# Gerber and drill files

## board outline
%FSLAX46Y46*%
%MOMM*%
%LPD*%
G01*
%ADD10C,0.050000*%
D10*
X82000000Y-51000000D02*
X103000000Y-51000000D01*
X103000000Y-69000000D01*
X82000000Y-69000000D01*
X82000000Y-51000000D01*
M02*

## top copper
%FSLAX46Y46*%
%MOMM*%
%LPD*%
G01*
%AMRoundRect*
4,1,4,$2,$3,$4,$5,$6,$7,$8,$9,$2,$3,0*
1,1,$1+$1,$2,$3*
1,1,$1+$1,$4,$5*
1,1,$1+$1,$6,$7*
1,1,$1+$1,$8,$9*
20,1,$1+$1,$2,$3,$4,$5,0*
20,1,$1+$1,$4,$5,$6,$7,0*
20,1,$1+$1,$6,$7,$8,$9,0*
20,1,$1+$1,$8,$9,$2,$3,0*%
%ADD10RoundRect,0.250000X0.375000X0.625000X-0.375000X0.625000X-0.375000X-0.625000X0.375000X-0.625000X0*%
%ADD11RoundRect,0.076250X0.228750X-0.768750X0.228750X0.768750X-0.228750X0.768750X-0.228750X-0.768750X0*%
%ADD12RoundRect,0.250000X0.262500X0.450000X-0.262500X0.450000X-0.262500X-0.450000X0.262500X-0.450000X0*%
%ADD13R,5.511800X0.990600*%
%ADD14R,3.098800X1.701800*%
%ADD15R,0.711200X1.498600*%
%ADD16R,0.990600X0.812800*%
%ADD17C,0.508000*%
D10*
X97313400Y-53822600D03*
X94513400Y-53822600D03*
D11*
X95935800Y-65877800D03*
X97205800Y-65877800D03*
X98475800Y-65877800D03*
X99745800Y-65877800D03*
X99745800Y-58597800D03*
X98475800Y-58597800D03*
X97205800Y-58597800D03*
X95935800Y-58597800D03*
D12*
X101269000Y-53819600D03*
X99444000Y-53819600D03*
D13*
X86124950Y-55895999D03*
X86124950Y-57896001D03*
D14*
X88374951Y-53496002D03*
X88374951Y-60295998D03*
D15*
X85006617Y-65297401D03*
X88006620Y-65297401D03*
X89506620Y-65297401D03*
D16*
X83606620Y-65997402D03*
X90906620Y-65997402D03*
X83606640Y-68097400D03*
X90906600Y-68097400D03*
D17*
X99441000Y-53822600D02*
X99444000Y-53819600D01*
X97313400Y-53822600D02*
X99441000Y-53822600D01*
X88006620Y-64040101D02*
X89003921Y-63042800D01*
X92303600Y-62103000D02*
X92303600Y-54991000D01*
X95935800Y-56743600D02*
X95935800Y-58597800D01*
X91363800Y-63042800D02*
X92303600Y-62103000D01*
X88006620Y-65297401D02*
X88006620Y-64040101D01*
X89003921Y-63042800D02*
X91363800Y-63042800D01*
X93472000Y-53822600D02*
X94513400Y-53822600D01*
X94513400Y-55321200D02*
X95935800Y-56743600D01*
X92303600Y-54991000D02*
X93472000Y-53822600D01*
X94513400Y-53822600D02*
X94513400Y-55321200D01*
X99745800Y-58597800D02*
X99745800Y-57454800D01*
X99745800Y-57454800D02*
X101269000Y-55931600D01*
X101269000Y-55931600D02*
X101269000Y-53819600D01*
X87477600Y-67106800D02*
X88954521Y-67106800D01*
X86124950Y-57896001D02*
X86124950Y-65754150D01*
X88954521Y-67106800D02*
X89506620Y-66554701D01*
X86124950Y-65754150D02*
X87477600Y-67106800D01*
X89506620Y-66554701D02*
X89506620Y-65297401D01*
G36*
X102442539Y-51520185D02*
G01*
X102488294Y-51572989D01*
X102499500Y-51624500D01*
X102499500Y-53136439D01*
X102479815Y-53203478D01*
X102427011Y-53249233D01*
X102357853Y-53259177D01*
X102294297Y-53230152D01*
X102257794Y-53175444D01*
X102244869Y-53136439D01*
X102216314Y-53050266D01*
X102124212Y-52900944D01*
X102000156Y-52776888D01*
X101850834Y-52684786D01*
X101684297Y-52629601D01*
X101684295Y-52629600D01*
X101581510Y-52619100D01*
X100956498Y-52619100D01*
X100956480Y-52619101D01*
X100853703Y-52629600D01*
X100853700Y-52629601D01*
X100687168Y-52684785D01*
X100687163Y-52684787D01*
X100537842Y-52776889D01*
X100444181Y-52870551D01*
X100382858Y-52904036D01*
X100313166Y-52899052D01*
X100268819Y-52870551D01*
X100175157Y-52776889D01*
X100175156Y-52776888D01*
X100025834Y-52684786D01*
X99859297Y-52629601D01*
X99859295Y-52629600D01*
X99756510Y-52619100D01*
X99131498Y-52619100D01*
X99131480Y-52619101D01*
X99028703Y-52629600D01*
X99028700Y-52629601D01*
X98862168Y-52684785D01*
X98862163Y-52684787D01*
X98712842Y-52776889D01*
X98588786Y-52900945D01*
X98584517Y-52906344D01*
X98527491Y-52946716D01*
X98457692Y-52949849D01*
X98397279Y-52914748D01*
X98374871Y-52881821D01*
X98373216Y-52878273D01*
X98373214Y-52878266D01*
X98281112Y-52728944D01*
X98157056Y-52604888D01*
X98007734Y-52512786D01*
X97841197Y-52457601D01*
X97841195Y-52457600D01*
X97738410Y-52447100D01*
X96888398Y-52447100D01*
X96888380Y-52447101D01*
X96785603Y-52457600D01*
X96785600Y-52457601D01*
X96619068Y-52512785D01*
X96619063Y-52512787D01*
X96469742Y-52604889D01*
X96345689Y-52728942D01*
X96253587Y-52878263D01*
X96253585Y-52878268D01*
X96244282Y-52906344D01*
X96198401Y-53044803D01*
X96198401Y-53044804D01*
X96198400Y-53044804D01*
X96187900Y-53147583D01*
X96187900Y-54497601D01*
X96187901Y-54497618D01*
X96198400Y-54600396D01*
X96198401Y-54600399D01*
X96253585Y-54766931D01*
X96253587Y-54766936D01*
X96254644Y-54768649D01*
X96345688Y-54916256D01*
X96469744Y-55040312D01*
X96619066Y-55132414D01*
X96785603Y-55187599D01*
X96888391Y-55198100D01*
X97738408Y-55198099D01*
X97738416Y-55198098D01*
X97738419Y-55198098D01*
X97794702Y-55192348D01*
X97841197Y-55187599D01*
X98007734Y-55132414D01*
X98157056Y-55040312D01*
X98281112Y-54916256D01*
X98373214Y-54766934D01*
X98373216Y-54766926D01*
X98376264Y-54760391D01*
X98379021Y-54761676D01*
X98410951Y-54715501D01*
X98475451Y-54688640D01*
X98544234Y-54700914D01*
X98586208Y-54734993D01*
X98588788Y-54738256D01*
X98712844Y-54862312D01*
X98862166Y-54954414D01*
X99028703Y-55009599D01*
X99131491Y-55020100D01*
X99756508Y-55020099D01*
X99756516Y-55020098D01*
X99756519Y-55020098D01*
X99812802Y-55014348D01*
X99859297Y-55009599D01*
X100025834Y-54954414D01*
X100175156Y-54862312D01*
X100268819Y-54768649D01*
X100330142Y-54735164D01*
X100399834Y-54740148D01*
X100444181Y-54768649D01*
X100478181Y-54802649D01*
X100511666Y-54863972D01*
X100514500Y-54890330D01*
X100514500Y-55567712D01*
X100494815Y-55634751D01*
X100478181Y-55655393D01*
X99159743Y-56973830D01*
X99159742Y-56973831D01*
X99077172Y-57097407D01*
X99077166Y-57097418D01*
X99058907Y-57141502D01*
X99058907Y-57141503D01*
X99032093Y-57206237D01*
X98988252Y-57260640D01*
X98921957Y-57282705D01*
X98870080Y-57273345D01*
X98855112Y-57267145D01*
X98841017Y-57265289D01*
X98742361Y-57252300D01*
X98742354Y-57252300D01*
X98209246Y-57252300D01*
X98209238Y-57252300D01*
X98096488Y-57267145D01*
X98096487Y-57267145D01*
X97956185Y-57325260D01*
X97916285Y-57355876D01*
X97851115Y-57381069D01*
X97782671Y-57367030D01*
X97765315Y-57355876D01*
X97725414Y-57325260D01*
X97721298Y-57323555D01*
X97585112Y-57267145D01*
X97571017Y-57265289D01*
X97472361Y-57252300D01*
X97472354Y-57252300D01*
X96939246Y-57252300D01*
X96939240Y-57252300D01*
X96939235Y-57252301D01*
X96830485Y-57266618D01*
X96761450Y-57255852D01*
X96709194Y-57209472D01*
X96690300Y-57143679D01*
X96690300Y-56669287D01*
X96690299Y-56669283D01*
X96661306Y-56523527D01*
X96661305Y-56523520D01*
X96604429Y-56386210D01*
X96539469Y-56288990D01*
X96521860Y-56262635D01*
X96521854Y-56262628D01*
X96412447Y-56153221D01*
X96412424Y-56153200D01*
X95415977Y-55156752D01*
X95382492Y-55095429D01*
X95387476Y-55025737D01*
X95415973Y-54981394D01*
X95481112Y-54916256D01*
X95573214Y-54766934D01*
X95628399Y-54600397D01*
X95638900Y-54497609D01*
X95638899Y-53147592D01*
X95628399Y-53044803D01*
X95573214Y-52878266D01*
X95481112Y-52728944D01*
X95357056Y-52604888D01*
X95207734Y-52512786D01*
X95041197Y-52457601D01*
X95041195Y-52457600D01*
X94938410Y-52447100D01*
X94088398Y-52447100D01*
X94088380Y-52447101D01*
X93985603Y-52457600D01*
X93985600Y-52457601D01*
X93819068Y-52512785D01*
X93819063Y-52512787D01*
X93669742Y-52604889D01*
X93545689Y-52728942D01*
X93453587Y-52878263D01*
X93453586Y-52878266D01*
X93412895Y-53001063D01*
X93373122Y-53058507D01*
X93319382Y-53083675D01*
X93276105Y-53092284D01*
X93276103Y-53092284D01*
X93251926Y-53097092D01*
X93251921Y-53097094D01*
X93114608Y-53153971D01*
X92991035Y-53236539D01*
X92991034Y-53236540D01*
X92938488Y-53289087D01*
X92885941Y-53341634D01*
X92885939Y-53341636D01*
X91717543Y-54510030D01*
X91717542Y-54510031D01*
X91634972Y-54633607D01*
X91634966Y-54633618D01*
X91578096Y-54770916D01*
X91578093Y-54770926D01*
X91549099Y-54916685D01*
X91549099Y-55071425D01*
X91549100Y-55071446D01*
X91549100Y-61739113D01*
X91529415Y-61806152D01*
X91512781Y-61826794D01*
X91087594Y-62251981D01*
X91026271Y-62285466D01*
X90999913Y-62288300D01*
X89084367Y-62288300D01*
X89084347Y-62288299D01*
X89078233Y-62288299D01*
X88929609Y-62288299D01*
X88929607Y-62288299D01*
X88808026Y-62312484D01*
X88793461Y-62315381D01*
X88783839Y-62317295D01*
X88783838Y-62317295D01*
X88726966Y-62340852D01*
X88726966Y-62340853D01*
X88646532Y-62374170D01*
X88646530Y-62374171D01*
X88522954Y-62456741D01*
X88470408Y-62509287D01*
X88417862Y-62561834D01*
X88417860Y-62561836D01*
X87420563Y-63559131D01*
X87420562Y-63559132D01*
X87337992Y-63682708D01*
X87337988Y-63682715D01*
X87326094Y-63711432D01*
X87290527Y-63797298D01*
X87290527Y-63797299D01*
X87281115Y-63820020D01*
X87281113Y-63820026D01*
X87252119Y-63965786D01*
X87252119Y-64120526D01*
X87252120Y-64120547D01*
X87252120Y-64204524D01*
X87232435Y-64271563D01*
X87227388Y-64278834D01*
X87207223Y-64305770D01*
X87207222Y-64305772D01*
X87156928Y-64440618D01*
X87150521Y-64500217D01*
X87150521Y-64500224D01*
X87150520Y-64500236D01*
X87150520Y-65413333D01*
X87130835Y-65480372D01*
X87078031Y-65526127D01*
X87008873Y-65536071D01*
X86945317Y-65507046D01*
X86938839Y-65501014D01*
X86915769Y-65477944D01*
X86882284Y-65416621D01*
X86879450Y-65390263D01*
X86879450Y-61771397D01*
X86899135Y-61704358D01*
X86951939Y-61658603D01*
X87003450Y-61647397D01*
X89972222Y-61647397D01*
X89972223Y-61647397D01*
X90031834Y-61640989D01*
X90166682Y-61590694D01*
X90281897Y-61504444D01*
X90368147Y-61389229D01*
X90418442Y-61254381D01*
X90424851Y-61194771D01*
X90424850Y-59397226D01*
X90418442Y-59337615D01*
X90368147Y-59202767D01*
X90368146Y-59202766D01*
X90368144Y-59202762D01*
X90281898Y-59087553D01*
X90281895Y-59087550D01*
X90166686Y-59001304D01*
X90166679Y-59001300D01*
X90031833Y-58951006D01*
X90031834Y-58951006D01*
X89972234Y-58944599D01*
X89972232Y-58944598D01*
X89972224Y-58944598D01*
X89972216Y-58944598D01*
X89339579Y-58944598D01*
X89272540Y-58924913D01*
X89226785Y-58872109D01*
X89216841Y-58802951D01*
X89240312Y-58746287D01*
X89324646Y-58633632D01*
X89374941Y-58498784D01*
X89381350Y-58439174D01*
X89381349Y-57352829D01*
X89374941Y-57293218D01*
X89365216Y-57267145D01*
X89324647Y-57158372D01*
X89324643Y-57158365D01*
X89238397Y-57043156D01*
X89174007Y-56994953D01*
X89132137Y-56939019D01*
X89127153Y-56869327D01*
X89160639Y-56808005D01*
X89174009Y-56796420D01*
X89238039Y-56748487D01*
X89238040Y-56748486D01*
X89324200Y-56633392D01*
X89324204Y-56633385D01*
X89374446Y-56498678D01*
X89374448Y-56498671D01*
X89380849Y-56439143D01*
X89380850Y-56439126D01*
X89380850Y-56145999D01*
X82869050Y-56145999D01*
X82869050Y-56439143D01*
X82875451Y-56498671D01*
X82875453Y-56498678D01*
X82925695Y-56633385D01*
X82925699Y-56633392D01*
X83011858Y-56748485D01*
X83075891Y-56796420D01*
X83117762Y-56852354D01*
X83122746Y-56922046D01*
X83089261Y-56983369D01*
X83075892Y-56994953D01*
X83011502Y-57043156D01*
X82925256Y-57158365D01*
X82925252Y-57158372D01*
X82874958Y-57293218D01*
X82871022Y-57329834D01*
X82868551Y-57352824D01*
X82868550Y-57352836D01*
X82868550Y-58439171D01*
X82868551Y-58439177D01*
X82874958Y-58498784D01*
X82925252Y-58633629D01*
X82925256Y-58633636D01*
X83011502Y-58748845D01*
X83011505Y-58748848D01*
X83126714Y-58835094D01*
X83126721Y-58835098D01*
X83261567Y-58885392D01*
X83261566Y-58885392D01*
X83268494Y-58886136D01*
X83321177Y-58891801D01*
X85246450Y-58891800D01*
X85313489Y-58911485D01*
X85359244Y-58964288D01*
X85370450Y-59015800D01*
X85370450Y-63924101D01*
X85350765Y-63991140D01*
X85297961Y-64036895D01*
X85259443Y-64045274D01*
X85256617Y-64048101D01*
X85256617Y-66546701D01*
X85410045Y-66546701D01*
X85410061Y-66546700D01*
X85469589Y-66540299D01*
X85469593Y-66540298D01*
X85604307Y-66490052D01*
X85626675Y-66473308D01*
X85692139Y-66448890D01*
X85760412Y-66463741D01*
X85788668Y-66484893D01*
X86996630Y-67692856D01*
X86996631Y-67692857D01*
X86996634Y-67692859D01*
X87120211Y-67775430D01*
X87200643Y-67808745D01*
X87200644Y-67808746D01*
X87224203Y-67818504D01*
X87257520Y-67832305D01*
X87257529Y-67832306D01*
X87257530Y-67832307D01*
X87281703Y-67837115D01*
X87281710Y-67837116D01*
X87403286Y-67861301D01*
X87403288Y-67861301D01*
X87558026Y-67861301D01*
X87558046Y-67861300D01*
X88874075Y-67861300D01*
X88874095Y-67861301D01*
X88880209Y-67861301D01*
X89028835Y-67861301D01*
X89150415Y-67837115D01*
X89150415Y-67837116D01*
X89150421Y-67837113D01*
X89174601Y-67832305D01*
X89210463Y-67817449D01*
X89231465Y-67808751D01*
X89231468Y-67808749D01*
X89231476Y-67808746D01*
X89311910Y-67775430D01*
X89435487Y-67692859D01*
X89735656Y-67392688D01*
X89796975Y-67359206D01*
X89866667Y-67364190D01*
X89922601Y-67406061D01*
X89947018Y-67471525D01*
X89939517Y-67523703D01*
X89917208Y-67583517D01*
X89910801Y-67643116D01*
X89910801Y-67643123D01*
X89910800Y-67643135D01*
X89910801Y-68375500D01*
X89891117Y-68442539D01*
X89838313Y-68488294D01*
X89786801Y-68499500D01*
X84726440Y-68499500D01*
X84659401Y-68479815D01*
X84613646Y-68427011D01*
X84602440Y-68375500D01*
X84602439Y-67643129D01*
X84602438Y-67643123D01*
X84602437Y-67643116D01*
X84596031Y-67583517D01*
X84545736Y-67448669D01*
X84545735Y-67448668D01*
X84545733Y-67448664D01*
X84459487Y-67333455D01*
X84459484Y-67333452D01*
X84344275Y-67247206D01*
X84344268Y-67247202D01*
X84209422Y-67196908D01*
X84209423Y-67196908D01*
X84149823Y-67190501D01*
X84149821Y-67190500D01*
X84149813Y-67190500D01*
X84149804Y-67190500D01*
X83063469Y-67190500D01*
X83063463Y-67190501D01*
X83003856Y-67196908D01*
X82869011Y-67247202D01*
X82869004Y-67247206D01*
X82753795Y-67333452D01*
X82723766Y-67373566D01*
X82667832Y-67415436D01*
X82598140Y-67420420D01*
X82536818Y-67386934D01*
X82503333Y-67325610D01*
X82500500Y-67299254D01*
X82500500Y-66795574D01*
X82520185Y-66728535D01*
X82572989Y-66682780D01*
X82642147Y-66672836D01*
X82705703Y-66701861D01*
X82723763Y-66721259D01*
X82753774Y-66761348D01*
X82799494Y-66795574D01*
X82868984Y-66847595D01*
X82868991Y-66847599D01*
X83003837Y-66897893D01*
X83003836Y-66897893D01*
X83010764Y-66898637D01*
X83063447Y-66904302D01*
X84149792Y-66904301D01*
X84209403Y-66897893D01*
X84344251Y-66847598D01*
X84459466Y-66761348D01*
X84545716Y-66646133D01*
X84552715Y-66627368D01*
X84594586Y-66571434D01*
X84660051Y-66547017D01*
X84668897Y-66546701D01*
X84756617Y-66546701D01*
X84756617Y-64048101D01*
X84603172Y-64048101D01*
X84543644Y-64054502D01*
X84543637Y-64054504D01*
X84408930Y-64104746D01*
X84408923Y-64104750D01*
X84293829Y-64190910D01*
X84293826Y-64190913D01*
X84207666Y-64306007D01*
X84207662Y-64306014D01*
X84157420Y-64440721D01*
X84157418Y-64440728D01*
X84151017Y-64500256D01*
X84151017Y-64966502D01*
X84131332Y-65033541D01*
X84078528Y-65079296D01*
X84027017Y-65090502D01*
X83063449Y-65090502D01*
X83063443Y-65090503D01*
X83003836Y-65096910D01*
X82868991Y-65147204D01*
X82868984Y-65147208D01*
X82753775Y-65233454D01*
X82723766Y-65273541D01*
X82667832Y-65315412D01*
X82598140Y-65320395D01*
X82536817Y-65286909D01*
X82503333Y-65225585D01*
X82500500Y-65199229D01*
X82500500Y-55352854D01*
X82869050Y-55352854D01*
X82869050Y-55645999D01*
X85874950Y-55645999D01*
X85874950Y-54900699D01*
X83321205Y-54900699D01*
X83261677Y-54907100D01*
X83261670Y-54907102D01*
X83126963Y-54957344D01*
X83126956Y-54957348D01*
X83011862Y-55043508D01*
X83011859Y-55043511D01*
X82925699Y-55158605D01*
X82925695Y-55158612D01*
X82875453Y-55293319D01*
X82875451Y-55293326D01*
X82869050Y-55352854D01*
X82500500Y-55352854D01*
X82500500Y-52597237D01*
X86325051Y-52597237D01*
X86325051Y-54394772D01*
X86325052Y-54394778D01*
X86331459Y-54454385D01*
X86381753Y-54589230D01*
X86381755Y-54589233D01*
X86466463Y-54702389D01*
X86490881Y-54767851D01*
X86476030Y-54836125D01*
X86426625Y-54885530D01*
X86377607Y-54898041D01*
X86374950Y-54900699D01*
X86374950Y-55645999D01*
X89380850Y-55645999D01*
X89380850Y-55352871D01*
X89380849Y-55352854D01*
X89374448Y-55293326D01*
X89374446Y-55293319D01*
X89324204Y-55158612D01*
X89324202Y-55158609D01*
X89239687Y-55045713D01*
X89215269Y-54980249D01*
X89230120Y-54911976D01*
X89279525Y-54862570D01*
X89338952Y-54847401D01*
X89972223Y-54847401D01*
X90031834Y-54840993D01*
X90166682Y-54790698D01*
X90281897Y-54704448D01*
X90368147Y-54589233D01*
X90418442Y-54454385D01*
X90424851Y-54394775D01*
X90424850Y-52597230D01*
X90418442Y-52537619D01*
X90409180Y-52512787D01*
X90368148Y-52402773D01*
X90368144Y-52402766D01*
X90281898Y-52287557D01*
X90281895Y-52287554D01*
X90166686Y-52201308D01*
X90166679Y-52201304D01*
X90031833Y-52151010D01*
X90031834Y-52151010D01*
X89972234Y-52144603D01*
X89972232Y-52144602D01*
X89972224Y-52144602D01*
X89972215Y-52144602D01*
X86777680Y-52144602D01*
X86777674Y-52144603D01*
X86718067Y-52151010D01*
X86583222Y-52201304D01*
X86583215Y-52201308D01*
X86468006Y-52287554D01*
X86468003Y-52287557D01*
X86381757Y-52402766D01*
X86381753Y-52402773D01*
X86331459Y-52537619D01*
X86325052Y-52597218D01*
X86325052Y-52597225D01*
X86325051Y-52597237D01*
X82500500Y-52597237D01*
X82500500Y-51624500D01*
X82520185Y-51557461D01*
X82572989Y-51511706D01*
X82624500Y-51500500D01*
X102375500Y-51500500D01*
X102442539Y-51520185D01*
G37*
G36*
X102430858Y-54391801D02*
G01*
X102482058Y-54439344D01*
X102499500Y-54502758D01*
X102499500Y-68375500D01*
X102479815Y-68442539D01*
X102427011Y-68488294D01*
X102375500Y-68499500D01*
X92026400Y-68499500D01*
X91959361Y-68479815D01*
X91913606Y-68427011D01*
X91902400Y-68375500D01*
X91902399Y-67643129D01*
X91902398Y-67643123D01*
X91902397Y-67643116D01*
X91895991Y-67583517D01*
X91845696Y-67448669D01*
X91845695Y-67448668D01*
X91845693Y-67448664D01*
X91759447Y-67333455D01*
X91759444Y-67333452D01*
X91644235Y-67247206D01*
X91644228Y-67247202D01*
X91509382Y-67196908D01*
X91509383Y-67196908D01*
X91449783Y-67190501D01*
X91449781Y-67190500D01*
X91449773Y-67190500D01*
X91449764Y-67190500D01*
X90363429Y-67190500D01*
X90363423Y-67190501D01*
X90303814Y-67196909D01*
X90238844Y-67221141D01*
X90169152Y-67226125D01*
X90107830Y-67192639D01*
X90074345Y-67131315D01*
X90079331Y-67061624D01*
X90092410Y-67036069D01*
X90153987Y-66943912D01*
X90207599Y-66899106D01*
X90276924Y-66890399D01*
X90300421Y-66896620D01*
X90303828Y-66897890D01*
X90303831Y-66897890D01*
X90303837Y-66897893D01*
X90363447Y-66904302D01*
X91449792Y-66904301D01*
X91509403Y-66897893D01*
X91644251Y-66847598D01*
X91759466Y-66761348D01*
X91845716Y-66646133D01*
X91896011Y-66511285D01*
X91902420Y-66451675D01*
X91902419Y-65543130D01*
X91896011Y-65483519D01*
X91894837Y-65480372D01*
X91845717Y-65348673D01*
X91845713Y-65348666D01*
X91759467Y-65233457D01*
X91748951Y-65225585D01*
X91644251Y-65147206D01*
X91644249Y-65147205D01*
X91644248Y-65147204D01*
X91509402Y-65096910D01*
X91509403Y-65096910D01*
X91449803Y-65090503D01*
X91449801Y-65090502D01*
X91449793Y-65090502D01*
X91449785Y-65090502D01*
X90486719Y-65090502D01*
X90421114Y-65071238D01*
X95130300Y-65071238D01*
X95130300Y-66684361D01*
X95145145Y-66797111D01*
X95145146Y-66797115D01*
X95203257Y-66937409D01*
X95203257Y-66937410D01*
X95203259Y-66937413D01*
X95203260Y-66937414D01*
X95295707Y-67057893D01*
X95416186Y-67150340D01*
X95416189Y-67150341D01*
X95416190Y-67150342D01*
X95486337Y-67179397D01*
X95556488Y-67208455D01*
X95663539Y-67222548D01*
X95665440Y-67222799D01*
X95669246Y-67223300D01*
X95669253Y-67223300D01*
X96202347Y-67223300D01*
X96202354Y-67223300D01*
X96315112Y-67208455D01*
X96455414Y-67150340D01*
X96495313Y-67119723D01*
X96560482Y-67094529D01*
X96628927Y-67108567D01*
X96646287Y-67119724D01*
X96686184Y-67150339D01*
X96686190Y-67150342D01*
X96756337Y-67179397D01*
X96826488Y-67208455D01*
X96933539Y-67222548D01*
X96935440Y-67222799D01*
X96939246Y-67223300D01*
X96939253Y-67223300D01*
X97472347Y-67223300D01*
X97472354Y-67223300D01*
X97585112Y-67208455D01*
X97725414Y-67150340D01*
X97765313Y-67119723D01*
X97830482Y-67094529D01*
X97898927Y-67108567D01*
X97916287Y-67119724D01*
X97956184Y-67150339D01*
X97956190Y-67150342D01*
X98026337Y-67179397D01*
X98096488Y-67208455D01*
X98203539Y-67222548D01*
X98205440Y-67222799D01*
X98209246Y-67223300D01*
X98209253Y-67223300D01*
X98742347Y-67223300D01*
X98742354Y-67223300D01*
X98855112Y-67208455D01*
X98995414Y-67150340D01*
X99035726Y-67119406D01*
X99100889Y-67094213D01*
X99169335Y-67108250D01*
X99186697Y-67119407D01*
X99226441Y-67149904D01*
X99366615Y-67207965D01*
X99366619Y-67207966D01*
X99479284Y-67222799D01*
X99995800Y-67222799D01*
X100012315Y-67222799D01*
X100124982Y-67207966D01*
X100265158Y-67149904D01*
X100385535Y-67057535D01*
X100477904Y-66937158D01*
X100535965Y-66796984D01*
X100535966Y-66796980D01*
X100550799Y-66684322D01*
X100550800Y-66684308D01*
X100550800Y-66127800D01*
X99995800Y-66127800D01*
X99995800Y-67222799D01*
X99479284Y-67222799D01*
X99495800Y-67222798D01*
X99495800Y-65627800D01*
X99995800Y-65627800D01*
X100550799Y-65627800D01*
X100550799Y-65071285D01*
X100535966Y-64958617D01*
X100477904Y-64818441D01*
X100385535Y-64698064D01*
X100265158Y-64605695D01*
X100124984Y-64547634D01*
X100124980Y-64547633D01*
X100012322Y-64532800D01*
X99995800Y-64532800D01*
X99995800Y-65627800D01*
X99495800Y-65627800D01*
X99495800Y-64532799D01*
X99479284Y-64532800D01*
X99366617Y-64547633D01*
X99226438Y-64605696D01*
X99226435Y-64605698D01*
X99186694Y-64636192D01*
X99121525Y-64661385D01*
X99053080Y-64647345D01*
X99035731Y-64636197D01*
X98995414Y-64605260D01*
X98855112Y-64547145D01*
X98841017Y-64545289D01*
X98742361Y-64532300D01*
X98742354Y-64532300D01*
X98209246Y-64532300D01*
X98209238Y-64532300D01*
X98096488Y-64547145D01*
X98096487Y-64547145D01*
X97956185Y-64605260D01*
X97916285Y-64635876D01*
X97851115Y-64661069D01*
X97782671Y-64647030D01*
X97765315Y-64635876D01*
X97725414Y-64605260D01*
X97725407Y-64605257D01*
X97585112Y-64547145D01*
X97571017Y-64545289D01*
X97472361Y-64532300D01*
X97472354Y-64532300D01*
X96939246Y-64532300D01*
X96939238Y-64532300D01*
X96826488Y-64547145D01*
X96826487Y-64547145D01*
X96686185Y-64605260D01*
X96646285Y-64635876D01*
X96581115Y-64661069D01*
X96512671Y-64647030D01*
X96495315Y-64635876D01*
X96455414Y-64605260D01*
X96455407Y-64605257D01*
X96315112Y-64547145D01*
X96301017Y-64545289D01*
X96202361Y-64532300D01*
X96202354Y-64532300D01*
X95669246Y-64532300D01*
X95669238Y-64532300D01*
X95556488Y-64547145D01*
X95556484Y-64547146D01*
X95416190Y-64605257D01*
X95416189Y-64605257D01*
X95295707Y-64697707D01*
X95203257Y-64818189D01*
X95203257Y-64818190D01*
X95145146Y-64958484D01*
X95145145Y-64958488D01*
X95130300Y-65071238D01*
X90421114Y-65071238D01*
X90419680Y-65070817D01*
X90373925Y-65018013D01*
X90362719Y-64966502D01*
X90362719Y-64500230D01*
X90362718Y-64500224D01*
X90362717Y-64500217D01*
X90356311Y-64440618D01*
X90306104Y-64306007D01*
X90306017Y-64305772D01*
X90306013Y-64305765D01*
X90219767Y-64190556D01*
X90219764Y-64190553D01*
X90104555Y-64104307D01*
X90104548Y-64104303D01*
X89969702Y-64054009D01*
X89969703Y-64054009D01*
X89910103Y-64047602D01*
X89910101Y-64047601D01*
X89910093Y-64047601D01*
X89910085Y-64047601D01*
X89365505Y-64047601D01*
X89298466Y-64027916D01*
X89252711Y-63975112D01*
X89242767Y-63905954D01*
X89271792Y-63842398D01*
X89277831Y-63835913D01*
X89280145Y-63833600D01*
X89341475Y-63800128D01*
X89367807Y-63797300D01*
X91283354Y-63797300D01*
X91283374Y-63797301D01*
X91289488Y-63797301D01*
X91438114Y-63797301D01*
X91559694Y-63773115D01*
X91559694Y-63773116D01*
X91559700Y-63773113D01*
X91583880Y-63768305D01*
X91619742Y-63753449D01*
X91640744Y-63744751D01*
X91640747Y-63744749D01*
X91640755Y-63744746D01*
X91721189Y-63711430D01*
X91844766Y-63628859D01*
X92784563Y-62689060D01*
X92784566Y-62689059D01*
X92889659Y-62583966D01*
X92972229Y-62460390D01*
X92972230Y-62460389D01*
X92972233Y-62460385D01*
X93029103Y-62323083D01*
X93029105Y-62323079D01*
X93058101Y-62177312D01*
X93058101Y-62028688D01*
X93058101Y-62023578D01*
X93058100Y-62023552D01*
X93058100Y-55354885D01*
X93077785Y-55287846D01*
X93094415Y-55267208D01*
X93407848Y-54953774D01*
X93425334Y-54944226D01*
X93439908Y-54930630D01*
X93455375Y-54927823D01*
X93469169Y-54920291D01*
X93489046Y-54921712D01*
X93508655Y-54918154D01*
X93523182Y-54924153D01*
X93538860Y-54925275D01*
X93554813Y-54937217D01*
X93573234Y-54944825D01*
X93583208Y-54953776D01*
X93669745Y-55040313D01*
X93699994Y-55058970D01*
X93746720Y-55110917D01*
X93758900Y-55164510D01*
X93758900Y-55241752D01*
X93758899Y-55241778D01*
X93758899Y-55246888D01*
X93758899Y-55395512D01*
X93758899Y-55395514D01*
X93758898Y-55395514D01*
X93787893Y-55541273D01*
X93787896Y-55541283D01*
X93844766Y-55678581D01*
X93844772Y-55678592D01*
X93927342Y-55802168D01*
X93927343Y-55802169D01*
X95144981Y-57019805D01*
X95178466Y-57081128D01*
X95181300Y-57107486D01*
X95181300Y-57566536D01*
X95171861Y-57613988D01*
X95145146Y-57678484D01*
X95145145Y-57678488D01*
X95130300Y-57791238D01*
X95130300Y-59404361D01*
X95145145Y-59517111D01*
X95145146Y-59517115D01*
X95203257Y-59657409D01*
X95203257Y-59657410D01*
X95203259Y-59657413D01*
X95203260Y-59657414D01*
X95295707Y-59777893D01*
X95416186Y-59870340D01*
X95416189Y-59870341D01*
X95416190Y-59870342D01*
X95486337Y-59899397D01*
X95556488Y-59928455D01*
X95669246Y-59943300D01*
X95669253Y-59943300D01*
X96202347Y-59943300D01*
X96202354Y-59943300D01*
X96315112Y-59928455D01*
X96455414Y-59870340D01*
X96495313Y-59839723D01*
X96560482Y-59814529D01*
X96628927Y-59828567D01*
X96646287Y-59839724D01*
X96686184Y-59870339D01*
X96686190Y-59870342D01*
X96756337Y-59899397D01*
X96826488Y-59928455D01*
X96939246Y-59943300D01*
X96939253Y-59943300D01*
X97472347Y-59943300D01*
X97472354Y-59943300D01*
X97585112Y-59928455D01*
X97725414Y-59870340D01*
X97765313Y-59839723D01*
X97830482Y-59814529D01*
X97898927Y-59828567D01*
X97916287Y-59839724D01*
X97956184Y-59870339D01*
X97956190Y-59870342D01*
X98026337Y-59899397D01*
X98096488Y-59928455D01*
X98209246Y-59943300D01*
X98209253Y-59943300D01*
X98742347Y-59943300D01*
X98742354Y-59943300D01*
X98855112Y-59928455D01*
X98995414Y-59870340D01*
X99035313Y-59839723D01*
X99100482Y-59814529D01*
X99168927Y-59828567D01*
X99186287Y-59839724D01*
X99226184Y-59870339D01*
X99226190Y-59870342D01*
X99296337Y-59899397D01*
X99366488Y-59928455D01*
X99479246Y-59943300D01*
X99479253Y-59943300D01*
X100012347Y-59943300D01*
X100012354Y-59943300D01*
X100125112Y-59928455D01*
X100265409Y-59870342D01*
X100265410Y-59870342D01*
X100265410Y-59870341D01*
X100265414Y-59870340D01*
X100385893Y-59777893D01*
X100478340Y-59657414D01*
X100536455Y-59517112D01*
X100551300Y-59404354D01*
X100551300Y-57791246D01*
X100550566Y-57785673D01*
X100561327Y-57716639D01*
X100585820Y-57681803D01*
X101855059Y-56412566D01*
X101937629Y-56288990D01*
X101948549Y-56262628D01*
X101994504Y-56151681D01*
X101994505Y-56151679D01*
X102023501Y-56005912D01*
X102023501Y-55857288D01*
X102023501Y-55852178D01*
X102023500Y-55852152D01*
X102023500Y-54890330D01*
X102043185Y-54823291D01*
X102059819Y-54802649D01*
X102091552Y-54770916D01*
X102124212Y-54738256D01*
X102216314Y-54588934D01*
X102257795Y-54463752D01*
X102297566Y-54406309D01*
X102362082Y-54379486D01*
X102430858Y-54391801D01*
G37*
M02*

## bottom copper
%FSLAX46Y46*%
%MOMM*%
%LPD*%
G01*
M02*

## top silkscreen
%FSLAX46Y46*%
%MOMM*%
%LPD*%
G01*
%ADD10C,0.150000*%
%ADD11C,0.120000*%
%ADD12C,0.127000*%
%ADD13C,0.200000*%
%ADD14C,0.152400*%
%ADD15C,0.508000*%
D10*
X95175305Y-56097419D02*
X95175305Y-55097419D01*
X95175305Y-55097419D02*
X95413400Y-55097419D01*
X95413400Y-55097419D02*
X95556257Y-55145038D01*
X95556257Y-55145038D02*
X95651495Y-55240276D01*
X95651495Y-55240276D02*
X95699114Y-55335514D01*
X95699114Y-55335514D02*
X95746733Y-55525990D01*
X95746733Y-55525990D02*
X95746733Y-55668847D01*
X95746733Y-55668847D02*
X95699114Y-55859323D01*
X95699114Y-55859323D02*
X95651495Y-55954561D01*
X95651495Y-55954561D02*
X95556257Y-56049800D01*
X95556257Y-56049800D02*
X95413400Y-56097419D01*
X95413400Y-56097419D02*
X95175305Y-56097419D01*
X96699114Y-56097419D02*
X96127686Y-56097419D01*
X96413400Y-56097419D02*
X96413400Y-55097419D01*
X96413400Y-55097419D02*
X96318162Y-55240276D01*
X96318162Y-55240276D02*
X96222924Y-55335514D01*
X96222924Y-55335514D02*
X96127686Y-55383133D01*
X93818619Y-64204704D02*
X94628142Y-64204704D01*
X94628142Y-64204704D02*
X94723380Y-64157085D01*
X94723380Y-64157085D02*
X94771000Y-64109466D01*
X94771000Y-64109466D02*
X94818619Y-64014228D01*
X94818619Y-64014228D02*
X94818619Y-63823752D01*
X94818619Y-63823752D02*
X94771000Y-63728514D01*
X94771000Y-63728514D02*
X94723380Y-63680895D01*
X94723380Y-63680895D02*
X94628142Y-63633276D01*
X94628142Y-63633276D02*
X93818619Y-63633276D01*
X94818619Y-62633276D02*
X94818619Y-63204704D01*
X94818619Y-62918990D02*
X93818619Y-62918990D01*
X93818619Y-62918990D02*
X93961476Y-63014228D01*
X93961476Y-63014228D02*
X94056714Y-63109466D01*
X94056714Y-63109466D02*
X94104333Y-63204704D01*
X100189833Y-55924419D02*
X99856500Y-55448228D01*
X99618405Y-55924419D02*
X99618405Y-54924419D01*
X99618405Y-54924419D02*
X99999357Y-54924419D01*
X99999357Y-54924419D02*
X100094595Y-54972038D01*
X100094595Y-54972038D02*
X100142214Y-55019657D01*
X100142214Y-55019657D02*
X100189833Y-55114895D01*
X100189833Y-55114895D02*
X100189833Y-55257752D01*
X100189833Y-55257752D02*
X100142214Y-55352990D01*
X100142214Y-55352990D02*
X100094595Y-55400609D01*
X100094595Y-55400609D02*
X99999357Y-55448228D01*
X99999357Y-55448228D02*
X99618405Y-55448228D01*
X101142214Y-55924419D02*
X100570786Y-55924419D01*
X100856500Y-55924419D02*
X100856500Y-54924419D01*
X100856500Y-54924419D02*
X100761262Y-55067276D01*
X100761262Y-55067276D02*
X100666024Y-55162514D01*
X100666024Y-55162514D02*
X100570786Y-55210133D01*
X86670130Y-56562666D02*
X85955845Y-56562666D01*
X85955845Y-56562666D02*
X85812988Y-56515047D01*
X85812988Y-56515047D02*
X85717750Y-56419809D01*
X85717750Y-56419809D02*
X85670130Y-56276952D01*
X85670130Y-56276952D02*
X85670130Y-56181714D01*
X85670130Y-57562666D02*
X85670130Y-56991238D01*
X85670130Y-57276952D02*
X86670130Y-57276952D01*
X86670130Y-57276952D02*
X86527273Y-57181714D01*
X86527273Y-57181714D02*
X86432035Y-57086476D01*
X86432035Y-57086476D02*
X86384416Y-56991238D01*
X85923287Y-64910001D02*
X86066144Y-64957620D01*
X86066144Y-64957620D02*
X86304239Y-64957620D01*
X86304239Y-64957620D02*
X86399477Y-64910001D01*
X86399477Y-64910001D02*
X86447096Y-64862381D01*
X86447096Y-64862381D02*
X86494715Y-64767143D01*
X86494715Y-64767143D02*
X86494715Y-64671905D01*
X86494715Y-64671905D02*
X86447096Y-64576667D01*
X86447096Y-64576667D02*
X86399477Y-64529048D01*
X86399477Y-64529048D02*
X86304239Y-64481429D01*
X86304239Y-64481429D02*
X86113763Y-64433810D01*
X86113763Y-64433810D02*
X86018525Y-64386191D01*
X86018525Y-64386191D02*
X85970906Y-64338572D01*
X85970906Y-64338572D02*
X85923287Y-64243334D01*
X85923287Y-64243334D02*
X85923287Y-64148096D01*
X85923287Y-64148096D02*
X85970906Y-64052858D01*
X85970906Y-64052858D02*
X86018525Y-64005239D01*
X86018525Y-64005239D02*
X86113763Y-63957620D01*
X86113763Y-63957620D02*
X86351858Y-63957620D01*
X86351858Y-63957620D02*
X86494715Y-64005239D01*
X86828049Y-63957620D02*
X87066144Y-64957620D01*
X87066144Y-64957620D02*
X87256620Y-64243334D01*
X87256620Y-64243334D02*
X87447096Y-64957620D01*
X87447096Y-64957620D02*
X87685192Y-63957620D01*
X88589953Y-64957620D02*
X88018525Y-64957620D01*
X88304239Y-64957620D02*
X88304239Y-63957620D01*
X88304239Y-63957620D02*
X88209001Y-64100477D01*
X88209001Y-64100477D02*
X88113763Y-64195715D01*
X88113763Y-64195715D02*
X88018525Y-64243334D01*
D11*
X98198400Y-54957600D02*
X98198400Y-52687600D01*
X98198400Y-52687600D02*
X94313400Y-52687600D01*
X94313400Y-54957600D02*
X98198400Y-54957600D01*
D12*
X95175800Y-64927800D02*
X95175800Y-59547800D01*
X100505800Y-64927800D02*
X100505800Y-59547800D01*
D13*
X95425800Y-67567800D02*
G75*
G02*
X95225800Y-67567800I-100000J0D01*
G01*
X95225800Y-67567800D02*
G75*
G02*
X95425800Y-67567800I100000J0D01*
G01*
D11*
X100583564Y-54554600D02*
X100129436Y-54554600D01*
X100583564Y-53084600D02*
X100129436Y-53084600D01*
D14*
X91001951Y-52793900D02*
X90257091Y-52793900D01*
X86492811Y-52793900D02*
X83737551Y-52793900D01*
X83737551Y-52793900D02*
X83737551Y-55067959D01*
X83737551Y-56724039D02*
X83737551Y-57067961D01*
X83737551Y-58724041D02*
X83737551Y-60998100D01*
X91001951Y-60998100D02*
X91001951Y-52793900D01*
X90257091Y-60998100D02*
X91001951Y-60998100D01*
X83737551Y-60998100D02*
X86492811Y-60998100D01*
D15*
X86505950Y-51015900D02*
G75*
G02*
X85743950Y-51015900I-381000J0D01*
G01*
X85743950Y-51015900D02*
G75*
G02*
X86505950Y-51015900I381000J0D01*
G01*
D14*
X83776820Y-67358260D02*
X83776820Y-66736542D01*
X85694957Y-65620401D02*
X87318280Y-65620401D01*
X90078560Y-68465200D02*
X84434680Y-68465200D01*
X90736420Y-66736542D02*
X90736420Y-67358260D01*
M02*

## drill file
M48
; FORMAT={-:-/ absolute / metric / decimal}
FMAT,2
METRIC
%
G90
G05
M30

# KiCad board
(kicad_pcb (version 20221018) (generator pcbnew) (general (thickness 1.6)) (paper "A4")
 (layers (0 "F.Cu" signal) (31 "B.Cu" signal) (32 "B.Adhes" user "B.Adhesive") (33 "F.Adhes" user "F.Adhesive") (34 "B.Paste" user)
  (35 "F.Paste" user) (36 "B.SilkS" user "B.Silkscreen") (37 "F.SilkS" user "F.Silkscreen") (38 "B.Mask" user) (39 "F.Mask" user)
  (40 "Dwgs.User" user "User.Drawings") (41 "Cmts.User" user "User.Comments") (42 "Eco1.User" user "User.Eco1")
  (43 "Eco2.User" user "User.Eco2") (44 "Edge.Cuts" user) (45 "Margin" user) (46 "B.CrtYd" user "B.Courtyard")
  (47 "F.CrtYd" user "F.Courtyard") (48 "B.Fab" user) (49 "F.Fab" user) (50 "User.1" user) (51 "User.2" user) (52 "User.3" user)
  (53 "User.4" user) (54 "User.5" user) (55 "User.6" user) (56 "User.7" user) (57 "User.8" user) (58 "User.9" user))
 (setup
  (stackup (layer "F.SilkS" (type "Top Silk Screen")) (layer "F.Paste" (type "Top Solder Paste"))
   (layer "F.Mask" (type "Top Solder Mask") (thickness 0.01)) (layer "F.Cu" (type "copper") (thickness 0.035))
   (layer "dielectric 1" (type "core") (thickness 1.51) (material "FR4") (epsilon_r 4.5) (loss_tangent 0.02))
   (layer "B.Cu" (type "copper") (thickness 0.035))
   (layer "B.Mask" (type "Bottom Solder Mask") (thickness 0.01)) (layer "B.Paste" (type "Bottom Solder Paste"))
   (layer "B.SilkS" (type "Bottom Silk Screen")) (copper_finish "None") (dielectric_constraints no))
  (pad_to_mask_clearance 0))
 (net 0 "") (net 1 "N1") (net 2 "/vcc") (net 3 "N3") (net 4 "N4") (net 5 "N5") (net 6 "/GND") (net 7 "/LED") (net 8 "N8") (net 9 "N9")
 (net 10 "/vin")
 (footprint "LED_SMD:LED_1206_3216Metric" (layer "F.Cu") (at 95.9134 53.8226 180)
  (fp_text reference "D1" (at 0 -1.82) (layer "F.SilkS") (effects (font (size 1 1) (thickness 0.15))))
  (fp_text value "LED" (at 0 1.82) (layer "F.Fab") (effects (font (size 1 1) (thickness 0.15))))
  (fp_line (start -2.285 -1.135) (end -2.285 1.135) (stroke (width 0.12) (type solid)) (layer "F.SilkS"))
  (fp_line (start -2.285 1.135) (end 1.6 1.135) (stroke (width 0.12) (type solid)) (layer "F.SilkS"))
  (fp_line (start 1.6 -1.135) (end -2.285 -1.135) (stroke (width 0.12) (type solid)) (layer "F.SilkS"))
  (pad "1" smd roundrect (at -1.4 0 180) (size 1.25 1.75) (layers "F.Cu" "F.Paste" "F.Mask") (roundrect_rratio 0.2) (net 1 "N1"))
  (pad "2" smd roundrect (at 1.4 0 180) (size 1.25 1.75) (layers "F.Cu" "F.Paste" "F.Mask") (roundrect_rratio 0.2) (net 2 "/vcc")))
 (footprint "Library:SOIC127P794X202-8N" (layer "F.Cu") (at 97.8408 62.2378 90)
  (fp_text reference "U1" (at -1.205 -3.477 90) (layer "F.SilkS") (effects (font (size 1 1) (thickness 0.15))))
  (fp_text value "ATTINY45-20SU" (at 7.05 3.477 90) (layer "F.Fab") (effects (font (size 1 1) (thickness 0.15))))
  (fp_line (start -2.69 -2.665) (end 2.69 -2.665) (stroke (width 0.127) (type solid)) (layer "F.SilkS"))
  (fp_line (start -2.69 2.665) (end 2.69 2.665) (stroke (width 0.127) (type solid)) (layer "F.SilkS"))
  (fp_circle (center -5.33 -2.515) (end -5.23 -2.515) (stroke (width 0.2) (type solid)) (fill none) (layer "F.SilkS"))
  (pad "1" smd roundrect (at -3.64 -1.905 90) (size 1.69 0.61) (layers "F.Cu" "F.Paste" "F.Mask") (roundrect_rratio 0.125) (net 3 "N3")
   (solder_mask_margin 0.102))
  (pad "2" smd roundrect (at -3.64 -0.635 90) (size 1.69 0.61) (layers "F.Cu" "F.Paste" "F.Mask") (roundrect_rratio 0.125) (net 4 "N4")
   (solder_mask_margin 0.102))
  (pad "3" smd roundrect (at -3.64 0.635 90) (size 1.69 0.61) (layers "F.Cu" "F.Paste" "F.Mask") (roundrect_rratio 0.125) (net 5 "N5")
   (solder_mask_margin 0.102))
  (pad "4" smd roundrect (at -3.64 1.905 90) (size 1.69 0.61) (layers "F.Cu" "F.Paste" "F.Mask") (roundrect_rratio 0.125) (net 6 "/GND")
   (solder_mask_margin 0.102))
  (pad "5" smd roundrect (at 3.64 1.905 90) (size 1.69 0.61) (layers "F.Cu" "F.Paste" "F.Mask") (roundrect_rratio 0.125) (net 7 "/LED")
   (solder_mask_margin 0.102))
  (pad "6" smd roundrect (at 3.64 0.635 90) (size 1.69 0.61) (layers "F.Cu" "F.Paste" "F.Mask") (roundrect_rratio 0.125) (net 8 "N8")
   (solder_mask_margin 0.102))
  (pad "7" smd roundrect (at 3.64 -0.635 90) (size 1.69 0.61) (layers "F.Cu" "F.Paste" "F.Mask") (roundrect_rratio 0.125) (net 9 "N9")
   (solder_mask_margin 0.102))
  (pad "8" smd roundrect (at 3.64 -1.905 90) (size 1.69 0.61) (layers "F.Cu" "F.Paste" "F.Mask") (roundrect_rratio 0.125) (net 2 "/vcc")
   (solder_mask_margin 0.102)))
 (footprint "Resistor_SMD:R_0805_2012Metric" (layer "F.Cu") (at 100.3565 53.8196 180)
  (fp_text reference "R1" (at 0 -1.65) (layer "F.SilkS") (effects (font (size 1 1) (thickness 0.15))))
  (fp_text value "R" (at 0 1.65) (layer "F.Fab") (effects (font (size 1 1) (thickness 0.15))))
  (fp_line (start -0.227064 -0.735) (end 0.227064 -0.735) (stroke (width 0.12) (type solid)) (layer "F.SilkS"))
  (fp_line (start -0.227064 0.735) (end 0.227064 0.735) (stroke (width 0.12) (type solid)) (layer "F.SilkS"))
  (pad "1" smd roundrect (at -0.9125 0 180) (size 1.025 1.4) (layers "F.Cu" "F.Paste" "F.Mask") (roundrect_rratio 0.243902439)
   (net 7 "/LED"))
  (pad "2" smd roundrect (at 0.9125 0 180) (size 1.025 1.4) (layers "F.Cu" "F.Paste" "F.Mask") (roundrect_rratio 0.243902439) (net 1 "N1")))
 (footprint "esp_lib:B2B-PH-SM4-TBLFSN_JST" (layer "F.Cu") (at 87.369751 56.896 -90)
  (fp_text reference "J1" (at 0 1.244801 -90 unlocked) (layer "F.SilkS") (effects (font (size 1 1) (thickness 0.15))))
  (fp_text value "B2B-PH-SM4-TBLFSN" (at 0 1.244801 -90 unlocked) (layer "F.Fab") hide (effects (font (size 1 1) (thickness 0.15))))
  (fp_line (start -4.1021 -3.6322) (end -4.1021 -2.88734) (stroke (width 0.1524) (type solid)) (layer "F.SilkS"))
  (fp_line (start -4.1021 0.87694) (end -4.1021 3.6322) (stroke (width 0.1524) (type solid)) (layer "F.SilkS"))
  (fp_line (start -4.1021 3.6322) (end -1.828041 3.6322) (stroke (width 0.1524) (type solid)) (layer "F.SilkS"))
  (fp_line (start -0.171961 3.6322) (end 0.171961 3.6322) (stroke (width 0.1524) (type solid)) (layer "F.SilkS"))
  (fp_line (start 1.828041 3.6322) (end 4.1021 3.6322) (stroke (width 0.1524) (type solid)) (layer "F.SilkS"))
  (fp_line (start 4.1021 -3.6322) (end -4.1021 -3.6322) (stroke (width 0.1524) (type solid)) (layer "F.SilkS"))
  (fp_line (start 4.1021 -2.88734) (end 4.1021 -3.6322) (stroke (width 0.1524) (type solid)) (layer "F.SilkS"))
  (fp_line (start 4.1021 3.6322) (end 4.1021 0.87694) (stroke (width 0.1524) (type solid)) (layer "F.SilkS"))
  (fp_circle (center -5.8801 1.244801) (end -5.4991 1.244801) (stroke (width 0.508) (type solid)) (fill none) (layer "F.SilkS"))
  (pad "1" smd rect (at -1.000001 1.244801 270) (size 0.9906 5.5118) (layers "F.Cu" "F.Paste" "F.Mask") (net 6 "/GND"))
  (pad "2" smd rect (at 1.000001 1.244801 270) (size 0.9906 5.5118) (layers "F.Cu" "F.Paste" "F.Mask") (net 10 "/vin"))
  (pad "3" smd rect (at -3.399998 -1.0052) (size 3.0988 1.7018) (layers "F.Cu" "F.Paste" "F.Mask"))
  (pad "4" smd rect (at 3.399998 -1.0052) (size 3.0988 1.7018) (layers "F.Cu" "F.Paste" "F.Mask")))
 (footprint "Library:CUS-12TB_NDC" (layer "F.Cu") (at 87.25662 67.042801)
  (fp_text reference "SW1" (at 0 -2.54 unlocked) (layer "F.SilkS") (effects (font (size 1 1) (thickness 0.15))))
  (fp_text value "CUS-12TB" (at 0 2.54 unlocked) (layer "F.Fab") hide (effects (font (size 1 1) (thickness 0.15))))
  (fp_line (start -3.4798 0.315459) (end -3.4798 -0.306259) (stroke (width 0.1524) (type solid)) (layer "F.SilkS"))
  (fp_line (start -1.561663 -1.4224) (end 0.06166 -1.4224) (stroke (width 0.1524) (type solid)) (layer "F.SilkS"))
  (fp_line (start 2.82194 1.422399) (end -2.82194 1.422399) (stroke (width 0.1524) (type solid)) (layer "F.SilkS"))
  (fp_line (start 3.4798 -0.306259) (end 3.4798 0.315459) (stroke (width 0.1524) (type solid)) (layer "F.SilkS"))
  (pad "1" smd rect (at -2.250003 -1.7454) (size 0.7112 1.4986) (layers "F.Cu" "F.Paste" "F.Mask") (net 6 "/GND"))
  (pad "2" smd rect (at 0.75 -1.7454) (size 0.7112 1.4986) (layers "F.Cu" "F.Paste" "F.Mask") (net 2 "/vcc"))
  (pad "3" smd rect (at 2.25 -1.7454) (size 0.7112 1.4986) (layers "F.Cu" "F.Paste" "F.Mask") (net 10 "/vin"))
  (pad "4" smd rect (at -3.65 -1.045399) (size 0.9906 0.8128) (layers "F.Cu" "F.Paste" "F.Mask"))
  (pad "5" smd rect (at 3.65 -1.045399) (size 0.9906 0.8128) (layers "F.Cu" "F.Paste" "F.Mask"))
  (pad "6" smd rect (at -3.64998 1.054599) (size 0.9906 0.8128) (layers "F.Cu" "F.Paste" "F.Mask"))
  (pad "7" smd rect (at 3.64998 1.054599) (size 0.9906 0.8128) (layers "F.Cu" "F.Paste" "F.Mask")))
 (gr_rect (start 82 51) (end 103 69) (stroke (width 0.05) (type default)) (fill none) (layer "Edge.Cuts"))
 (segment (start 99.441 53.8226) (end 99.444 53.8196) (width 0.508) (layer "F.Cu") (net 1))
 (segment (start 97.3134 53.8226) (end 99.441 53.8226) (width 0.508) (layer "F.Cu") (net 1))
 (segment (start 88.00662 64.040101) (end 89.003921 63.0428) (width 0.508) (layer "F.Cu") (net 2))
 (segment (start 92.3036 62.103) (end 92.3036 54.991) (width 0.508) (layer "F.Cu") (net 2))
 (segment (start 95.9358 56.7436) (end 95.9358 58.5978) (width 0.508) (layer "F.Cu") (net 2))
 (segment (start 91.3638 63.0428) (end 92.3036 62.103) (width 0.508) (layer "F.Cu") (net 2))
 (segment (start 88.00662 65.297401) (end 88.00662 64.040101) (width 0.508) (layer "F.Cu") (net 2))
 (segment (start 89.003921 63.0428) (end 91.3638 63.0428) (width 0.508) (layer "F.Cu") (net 2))
 (segment (start 93.472 53.8226) (end 94.5134 53.8226) (width 0.508) (layer "F.Cu") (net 2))
 (segment (start 94.5134 55.3212) (end 95.9358 56.7436) (width 0.508) (layer "F.Cu") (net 2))
 (segment (start 92.3036 54.991) (end 93.472 53.8226) (width 0.508) (layer "F.Cu") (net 2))
 (segment (start 94.5134 53.8226) (end 94.5134 55.3212) (width 0.508) (layer "F.Cu") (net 2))
 (segment (start 99.7458 58.5978) (end 99.7458 57.4548) (width 0.508) (layer "F.Cu") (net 7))
 (segment (start 99.7458 57.4548) (end 101.269 55.9316) (width 0.508) (layer "F.Cu") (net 7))
 (segment (start 101.269 55.9316) (end 101.269 53.8196) (width 0.508) (layer "F.Cu") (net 7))
 (segment (start 87.4776 67.1068) (end 88.954521 67.1068) (width 0.508) (layer "F.Cu") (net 10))
 (segment (start 86.12495 57.896001) (end 86.12495 65.75415) (width 0.508) (layer "F.Cu") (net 10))
 (segment (start 88.954521 67.1068) (end 89.50662 66.554701) (width 0.508) (layer "F.Cu") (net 10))
 (segment (start 86.12495 65.75415) (end 87.4776 67.1068) (width 0.508) (layer "F.Cu") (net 10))
 (segment (start 89.50662 66.554701) (end 89.50662 65.297401) (width 0.508) (layer "F.Cu") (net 10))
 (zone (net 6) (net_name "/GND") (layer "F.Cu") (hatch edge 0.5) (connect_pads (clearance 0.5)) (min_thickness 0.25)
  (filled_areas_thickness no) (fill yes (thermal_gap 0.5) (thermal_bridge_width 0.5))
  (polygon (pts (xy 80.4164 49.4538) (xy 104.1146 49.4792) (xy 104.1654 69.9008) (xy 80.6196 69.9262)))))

